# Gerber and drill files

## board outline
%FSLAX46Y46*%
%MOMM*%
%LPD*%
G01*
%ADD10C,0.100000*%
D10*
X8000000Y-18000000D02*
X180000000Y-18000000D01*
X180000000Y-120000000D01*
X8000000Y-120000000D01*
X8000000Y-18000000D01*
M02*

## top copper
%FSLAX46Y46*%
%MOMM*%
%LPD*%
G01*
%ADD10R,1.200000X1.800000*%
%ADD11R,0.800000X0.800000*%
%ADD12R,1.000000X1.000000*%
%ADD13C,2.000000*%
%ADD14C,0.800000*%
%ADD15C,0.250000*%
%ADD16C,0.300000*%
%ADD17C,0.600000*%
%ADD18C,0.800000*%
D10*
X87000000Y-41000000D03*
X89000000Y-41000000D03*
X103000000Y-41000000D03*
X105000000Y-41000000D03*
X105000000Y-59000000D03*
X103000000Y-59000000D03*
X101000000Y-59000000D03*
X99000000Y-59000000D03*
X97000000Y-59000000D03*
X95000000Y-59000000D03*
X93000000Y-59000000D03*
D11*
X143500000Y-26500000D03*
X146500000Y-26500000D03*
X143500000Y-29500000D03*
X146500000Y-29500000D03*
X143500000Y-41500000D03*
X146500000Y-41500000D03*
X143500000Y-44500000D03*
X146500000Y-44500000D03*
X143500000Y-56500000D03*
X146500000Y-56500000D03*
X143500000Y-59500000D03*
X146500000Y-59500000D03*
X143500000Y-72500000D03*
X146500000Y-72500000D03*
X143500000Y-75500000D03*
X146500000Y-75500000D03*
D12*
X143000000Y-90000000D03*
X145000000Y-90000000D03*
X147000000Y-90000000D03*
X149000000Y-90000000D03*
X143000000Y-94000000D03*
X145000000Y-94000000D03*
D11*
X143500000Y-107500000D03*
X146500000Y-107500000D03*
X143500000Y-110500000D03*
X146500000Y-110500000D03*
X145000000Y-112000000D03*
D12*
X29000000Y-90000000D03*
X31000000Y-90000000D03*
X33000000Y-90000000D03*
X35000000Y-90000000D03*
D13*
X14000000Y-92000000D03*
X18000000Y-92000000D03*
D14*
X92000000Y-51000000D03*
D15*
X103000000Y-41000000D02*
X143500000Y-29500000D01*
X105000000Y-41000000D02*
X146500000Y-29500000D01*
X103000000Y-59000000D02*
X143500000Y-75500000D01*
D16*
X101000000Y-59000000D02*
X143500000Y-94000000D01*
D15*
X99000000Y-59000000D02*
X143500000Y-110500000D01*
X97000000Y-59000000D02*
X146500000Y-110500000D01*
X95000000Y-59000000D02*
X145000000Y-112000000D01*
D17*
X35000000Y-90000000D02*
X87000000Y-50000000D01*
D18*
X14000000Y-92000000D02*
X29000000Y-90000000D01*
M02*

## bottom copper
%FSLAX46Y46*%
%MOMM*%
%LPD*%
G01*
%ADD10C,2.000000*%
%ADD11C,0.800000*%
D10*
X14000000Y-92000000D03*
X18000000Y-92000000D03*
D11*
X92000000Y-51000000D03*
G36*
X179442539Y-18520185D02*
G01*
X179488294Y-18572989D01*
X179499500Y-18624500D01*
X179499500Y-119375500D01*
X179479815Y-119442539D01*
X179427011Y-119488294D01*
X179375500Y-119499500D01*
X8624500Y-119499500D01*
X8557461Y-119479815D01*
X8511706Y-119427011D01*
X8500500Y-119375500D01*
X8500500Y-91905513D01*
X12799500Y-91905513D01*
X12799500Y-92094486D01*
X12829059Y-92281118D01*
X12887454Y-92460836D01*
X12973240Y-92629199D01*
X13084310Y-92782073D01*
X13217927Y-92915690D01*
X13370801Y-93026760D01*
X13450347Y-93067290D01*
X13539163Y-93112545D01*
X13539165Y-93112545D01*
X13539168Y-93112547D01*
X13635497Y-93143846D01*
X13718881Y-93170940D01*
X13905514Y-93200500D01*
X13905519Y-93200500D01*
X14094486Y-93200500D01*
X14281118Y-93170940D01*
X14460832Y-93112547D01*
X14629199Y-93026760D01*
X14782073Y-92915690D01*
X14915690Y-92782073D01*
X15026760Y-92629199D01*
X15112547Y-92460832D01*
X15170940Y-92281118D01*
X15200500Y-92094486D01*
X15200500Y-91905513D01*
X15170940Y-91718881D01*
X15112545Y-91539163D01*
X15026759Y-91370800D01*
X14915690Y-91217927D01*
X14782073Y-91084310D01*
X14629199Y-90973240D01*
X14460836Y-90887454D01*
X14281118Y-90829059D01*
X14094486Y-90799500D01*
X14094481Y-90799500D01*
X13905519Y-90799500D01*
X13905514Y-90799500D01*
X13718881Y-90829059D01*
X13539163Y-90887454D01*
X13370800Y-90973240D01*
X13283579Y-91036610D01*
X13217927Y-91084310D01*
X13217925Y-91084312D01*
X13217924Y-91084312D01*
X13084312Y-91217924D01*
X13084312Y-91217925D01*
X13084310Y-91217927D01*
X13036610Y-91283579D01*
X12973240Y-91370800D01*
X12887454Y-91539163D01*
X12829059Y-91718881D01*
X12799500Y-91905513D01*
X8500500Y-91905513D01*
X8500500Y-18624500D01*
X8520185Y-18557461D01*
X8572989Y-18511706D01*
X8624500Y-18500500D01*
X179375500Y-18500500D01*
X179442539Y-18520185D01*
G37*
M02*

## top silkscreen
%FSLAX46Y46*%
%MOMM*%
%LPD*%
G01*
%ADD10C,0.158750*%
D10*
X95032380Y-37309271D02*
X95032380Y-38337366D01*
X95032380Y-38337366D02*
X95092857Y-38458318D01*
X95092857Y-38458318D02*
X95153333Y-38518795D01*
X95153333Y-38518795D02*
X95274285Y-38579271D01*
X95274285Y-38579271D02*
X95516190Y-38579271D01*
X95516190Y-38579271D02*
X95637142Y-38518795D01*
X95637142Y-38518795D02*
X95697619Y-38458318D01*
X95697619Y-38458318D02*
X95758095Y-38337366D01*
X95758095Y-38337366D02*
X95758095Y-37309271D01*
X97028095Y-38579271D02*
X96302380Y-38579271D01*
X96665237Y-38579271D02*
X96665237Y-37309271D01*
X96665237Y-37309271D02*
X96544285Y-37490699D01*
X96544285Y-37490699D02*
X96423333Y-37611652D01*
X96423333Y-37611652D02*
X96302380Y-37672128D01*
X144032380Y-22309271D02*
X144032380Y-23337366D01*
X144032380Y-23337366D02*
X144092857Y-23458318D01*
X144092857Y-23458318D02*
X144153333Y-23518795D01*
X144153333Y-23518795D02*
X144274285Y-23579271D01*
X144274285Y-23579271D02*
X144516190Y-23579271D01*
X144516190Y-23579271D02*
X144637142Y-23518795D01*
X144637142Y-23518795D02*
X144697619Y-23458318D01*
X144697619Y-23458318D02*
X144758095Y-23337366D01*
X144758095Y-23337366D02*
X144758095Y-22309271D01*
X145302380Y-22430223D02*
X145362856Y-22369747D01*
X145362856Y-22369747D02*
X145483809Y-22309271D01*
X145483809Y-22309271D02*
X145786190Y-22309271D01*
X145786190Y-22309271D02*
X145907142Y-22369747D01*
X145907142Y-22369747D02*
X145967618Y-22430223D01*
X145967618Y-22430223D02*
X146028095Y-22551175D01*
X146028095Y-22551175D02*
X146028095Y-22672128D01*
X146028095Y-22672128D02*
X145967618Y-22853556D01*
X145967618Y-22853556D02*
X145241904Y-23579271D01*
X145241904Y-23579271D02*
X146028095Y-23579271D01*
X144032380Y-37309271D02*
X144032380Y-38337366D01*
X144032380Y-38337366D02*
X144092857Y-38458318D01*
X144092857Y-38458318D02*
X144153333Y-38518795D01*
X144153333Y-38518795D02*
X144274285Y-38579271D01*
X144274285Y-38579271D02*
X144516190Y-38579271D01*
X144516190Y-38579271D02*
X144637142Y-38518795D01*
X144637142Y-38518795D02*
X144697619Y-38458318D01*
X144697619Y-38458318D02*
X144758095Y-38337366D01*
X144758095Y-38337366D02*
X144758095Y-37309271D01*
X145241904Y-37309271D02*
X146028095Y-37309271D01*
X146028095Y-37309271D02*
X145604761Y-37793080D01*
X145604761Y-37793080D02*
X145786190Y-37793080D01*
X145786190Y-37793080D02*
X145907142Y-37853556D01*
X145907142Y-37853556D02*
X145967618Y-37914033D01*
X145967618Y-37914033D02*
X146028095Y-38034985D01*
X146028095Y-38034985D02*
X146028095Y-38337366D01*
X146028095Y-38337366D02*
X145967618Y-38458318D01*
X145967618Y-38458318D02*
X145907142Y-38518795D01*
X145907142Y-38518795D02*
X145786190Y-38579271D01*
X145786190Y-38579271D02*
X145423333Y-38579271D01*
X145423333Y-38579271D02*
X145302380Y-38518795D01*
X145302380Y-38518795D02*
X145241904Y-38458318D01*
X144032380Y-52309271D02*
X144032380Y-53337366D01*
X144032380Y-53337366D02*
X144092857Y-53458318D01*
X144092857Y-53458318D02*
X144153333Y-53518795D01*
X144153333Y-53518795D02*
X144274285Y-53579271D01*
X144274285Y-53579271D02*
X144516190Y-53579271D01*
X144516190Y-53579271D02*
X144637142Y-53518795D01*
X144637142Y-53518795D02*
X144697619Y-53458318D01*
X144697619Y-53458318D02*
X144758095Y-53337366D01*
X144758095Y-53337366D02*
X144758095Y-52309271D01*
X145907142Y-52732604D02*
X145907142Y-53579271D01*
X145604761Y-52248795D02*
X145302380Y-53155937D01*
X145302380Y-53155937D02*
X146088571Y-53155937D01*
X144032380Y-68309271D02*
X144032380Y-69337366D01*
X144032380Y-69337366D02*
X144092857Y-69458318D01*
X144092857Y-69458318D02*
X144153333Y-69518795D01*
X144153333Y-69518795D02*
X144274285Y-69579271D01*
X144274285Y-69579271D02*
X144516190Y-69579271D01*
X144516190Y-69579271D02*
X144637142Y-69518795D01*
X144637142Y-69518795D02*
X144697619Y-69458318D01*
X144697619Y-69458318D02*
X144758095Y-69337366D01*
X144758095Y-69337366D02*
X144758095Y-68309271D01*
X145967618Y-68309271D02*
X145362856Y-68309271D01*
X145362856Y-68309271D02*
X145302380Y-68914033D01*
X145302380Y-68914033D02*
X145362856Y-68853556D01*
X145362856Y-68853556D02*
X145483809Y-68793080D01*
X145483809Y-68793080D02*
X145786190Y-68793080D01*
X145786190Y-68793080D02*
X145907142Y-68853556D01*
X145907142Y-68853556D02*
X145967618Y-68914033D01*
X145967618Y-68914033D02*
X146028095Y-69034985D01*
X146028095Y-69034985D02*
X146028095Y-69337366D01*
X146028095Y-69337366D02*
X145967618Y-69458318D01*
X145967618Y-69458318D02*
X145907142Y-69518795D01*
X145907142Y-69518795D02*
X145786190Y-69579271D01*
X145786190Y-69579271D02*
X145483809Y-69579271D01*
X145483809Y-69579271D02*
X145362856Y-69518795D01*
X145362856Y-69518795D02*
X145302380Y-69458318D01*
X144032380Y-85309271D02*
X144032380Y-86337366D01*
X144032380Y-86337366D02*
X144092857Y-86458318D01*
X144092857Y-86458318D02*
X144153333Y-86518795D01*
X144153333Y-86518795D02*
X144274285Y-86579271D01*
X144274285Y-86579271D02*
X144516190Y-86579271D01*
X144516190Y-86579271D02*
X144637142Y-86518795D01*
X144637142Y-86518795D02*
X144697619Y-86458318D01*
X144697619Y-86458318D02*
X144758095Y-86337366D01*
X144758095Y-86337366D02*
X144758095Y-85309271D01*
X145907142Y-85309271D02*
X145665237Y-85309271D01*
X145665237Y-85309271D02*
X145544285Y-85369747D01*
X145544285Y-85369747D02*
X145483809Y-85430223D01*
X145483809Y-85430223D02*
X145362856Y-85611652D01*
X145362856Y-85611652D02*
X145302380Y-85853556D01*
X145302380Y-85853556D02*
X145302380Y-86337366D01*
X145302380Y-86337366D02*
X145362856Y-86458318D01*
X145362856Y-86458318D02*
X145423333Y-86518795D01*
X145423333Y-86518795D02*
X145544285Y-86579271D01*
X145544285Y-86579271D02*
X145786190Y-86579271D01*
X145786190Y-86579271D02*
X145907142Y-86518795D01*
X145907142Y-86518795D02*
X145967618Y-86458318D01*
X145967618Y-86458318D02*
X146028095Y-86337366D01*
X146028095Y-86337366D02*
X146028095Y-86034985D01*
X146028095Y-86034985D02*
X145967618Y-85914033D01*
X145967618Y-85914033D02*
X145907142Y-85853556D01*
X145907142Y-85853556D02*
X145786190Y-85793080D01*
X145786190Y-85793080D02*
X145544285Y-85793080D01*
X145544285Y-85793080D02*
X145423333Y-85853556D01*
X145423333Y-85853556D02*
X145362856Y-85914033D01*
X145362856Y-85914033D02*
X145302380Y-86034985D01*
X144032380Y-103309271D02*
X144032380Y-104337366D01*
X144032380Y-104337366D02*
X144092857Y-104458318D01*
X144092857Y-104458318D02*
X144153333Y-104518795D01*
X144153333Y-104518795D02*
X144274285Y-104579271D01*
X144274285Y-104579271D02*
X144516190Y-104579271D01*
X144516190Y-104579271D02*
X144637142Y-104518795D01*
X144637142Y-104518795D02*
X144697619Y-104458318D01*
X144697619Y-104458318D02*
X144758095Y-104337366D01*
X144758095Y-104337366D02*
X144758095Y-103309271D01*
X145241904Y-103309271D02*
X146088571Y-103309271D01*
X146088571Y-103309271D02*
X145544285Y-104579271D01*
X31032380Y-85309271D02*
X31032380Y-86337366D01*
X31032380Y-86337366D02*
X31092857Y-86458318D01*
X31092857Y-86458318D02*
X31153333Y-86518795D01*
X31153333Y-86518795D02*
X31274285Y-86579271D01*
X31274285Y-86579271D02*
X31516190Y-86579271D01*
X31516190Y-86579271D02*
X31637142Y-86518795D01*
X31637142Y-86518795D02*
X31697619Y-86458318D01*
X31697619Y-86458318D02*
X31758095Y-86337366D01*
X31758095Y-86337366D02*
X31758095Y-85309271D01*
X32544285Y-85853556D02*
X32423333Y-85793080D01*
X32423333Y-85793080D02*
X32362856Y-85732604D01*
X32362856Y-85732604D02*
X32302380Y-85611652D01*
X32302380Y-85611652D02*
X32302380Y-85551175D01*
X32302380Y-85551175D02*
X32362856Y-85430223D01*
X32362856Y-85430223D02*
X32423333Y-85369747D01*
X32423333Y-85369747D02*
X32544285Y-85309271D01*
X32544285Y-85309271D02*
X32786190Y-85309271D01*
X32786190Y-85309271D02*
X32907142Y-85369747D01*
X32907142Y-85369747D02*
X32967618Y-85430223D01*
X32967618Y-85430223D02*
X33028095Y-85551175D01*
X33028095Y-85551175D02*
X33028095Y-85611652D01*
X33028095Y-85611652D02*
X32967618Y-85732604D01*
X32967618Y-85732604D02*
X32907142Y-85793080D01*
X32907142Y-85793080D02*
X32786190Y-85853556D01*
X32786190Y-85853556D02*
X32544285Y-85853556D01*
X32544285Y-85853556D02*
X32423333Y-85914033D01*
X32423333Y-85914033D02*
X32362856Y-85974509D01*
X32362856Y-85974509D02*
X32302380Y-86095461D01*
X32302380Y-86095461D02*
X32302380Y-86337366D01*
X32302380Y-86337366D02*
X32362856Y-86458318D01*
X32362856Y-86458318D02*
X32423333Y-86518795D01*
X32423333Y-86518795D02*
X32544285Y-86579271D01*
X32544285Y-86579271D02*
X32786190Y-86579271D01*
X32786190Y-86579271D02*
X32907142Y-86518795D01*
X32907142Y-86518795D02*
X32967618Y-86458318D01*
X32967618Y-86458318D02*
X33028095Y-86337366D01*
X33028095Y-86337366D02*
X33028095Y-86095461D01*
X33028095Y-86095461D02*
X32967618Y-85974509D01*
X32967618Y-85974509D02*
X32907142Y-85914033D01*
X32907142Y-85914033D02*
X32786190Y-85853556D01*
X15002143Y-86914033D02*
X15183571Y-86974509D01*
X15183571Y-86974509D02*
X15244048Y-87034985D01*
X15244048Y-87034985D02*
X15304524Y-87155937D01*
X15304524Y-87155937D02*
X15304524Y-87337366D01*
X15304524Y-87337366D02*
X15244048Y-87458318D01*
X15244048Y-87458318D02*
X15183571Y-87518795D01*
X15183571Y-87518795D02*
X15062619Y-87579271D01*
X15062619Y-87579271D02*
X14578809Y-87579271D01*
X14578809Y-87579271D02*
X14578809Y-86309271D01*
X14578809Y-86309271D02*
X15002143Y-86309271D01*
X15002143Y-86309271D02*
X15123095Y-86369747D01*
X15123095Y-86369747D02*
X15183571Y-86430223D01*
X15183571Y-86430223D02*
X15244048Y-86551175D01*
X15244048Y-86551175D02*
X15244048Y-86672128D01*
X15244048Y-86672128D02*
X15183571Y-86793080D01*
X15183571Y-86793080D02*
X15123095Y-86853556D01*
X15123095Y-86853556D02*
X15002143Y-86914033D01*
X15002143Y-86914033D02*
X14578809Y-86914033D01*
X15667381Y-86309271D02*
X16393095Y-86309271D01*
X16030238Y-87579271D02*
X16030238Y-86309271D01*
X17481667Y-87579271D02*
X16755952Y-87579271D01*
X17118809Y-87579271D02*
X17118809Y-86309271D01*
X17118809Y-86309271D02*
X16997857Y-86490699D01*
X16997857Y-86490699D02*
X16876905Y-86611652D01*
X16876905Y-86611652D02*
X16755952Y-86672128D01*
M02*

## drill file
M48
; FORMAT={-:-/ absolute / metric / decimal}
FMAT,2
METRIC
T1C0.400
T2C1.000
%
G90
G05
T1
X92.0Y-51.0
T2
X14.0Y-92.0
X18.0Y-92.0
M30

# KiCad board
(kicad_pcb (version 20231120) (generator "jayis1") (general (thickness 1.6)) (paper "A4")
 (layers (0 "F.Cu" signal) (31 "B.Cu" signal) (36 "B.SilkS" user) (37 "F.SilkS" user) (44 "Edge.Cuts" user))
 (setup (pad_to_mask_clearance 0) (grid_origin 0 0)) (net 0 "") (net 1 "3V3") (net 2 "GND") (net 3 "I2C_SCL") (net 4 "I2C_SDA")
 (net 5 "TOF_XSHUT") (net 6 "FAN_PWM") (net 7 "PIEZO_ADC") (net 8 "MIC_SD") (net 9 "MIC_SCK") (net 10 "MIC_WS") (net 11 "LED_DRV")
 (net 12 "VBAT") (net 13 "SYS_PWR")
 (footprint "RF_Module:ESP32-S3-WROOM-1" (layer "F.Cu") (at 96 50) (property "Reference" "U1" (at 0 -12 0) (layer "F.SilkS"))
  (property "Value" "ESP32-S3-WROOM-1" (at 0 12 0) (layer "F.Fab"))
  (pad "1" smd rect (at -9 -9) (size 1.2 1.8) (layers "F.Cu" "F.Mask") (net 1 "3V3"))
  (pad "2" smd rect (at -7 -9) (size 1.2 1.8) (layers "F.Cu" "F.Mask") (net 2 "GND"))
  (pad "3" smd rect (at 7 -9) (size 1.2 1.8) (layers "F.Cu" "F.Mask") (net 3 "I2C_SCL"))
  (pad "4" smd rect (at 9 -9) (size 1.2 1.8) (layers "F.Cu" "F.Mask") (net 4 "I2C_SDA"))
  (pad "5" smd rect (at 9 9) (size 1.2 1.8) (layers "F.Cu" "F.Mask") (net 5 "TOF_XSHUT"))
  (pad "6" smd rect (at 7 9) (size 1.2 1.8) (layers "F.Cu" "F.Mask") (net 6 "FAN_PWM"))
  (pad "7" smd rect (at 5 9) (size 1.2 1.8) (layers "F.Cu" "F.Mask") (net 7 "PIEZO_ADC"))
  (pad "8" smd rect (at 3 9) (size 1.2 1.8) (layers "F.Cu" "F.Mask") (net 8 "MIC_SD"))
  (pad "9" smd rect (at 1 9) (size 1.2 1.8) (layers "F.Cu" "F.Mask") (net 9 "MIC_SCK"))
  (pad "10" smd rect (at -1 9) (size 1.2 1.8) (layers "F.Cu" "F.Mask") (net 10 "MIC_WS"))
  (pad "11" smd rect (at -3 9) (size 1.2 1.8) (layers "F.Cu" "F.Mask") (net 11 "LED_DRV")))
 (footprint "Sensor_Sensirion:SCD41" (layer "F.Cu") (at 145 28) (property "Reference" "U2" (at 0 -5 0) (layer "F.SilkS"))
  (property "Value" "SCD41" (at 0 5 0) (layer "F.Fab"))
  (pad "1" smd rect (at -1.5 -1.5) (size 0.8 0.8) (layers "F.Cu" "F.Mask") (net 1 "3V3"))
  (pad "2" smd rect (at 1.5 -1.5) (size 0.8 0.8) (layers "F.Cu" "F.Mask") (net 2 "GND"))
  (pad "3" smd rect (at -1.5 1.5) (size 0.8 0.8) (layers "F.Cu" "F.Mask") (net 3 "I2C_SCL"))
  (pad "4" smd rect (at 1.5 1.5) (size 0.8 0.8) (layers "F.Cu" "F.Mask") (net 4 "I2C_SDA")))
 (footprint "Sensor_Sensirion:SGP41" (layer "F.Cu") (at 145 43) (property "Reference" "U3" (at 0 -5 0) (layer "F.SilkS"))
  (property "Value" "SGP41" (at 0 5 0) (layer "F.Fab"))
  (pad "1" smd rect (at -1.5 -1.5) (size 0.8 0.8) (layers "F.Cu" "F.Mask") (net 1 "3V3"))
  (pad "2" smd rect (at 1.5 -1.5) (size 0.8 0.8) (layers "F.Cu" "F.Mask") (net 2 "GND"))
  (pad "3" smd rect (at -1.5 1.5) (size 0.8 0.8) (layers "F.Cu" "F.Mask") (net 3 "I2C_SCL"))
  (pad "4" smd rect (at 1.5 1.5) (size 0.8 0.8) (layers "F.Cu" "F.Mask") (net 4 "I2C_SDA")))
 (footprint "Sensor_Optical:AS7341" (layer "F.Cu") (at 145 58) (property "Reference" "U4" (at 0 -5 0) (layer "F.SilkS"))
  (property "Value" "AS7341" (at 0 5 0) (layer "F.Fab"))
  (pad "1" smd rect (at -1.5 -1.5) (size 0.8 0.8) (layers "F.Cu" "F.Mask") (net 1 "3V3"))
  (pad "2" smd rect (at 1.5 -1.5) (size 0.8 0.8) (layers "F.Cu" "F.Mask") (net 2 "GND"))
  (pad "3" smd rect (at -1.5 1.5) (size 0.8 0.8) (layers "F.Cu" "F.Mask") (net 3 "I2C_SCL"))
  (pad "4" smd rect (at 1.5 1.5) (size 0.8 0.8) (layers "F.Cu" "F.Mask") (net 4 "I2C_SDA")))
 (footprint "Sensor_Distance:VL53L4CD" (layer "F.Cu") (at 145 74) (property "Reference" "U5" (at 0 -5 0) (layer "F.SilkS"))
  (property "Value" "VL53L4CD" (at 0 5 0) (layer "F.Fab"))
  (pad "1" smd rect (at -1.5 -1.5) (size 0.8 0.8) (layers "F.Cu" "F.Mask") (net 1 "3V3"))
  (pad "2" smd rect (at 1.5 -1.5) (size 0.8 0.8) (layers "F.Cu" "F.Mask") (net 2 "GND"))
  (pad "3" smd rect (at -1.5 1.5) (size 0.8 0.8) (layers "F.Cu" "F.Mask") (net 3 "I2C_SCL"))
  (pad "4" smd rect (at 1.5 1.5) (size 0.8 0.8) (layers "F.Cu" "F.Mask") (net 4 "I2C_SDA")))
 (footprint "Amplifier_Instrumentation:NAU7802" (layer "F.Cu") (at 145 92) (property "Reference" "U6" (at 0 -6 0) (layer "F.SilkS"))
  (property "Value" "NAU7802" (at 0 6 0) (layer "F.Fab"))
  (pad "1" smd rect (at -2 -2) (size 1 1) (layers "F.Cu" "F.Mask") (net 1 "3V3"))
  (pad "2" smd rect (at 0 -2) (size 1 1) (layers "F.Cu" "F.Mask") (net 2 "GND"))
  (pad "3" smd rect (at 2 -2) (size 1 1) (layers "F.Cu" "F.Mask") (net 3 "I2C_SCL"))
  (pad "4" smd rect (at 4 -2) (size 1 1) (layers "F.Cu" "F.Mask") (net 4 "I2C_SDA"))
  (pad "5" smd rect (at -2 2) (size 1 1) (layers "F.Cu" "F.Mask") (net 7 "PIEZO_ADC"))
  (pad "6" smd rect (at 0 2) (size 1 1) (layers "F.Cu" "F.Mask") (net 2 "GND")))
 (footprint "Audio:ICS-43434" (layer "F.Cu") (at 145 109) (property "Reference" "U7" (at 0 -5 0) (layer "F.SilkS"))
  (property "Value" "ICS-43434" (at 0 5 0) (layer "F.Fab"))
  (pad "1" smd rect (at -1.5 -1.5) (size 0.8 0.8) (layers "F.Cu" "F.Mask") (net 1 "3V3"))
  (pad "2" smd rect (at 1.5 -1.5) (size 0.8 0.8) (layers "F.Cu" "F.Mask") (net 2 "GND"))
  (pad "3" smd rect (at -1.5 1.5) (size 0.8 0.8) (layers "F.Cu" "F.Mask") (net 8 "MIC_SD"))
  (pad "4" smd rect (at 1.5 1.5) (size 0.8 0.8) (layers "F.Cu" "F.Mask") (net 9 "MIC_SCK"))
  (pad "5" smd rect (at 0 3.0) (size 0.8 0.8) (layers "F.Cu" "F.Mask") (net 10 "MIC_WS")))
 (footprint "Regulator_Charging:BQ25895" (layer "F.Cu") (at 32 92) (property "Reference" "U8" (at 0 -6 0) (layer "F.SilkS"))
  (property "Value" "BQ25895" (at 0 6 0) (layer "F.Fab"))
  (pad "1" smd rect (at -3 -2) (size 1 1) (layers "F.Cu" "F.Mask") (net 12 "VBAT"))
  (pad "2" smd rect (at -1 -2) (size 1 1) (layers "F.Cu" "F.Mask") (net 12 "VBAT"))
  (pad "3" smd rect (at 1 -2) (size 1 1) (layers "F.Cu" "F.Mask") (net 2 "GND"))
  (pad "4" smd rect (at 3 -2) (size 1 1) (layers "F.Cu" "F.Mask") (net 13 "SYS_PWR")))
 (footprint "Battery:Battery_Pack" (layer "F.Cu") (at 16 92) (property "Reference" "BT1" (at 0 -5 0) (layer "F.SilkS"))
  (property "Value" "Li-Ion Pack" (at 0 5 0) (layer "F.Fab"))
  (pad "1" thru_hole circle (at -2 0) (size 2 2) (drill 1.0) (layers *.Cu *.Mask) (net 12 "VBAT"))
  (pad "2" thru_hole circle (at 2 0) (size 2 2) (drill 1.0) (layers *.Cu *.Mask) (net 2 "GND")))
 (gr_rect (start 8 18) (end 180 120) (stroke (width 0.1) (type default)) (fill none) (layer "Edge.Cuts"))
 (segment (start 103 41) (end 143.5 29.5) (width 0.25) (layer "F.Cu") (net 3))
 (segment (start 105 41) (end 146.5 29.5) (width 0.25) (layer "F.Cu") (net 4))
 (segment (start 103 59) (end 143.5 75.5) (width 0.25) (layer "F.Cu") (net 5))
 (segment (start 101 59) (end 143.5 94.0) (width 0.30) (layer "F.Cu") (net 7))
 (segment (start 99 59) (end 143.5 110.5) (width 0.25) (layer "F.Cu") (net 8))
 (segment (start 97 59) (end 146.5 110.5) (width 0.25) (layer "F.Cu") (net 9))
 (segment (start 95 59) (end 145 112.0) (width 0.25) (layer "F.Cu") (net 10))
 (segment (start 35 90) (end 87 50) (width 0.6) (layer "F.Cu") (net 13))
 (segment (start 14 92) (end 29 90) (width 0.8) (layer "F.Cu") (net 12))
 (via (at 92 51) (size 0.8) (drill 0.4) (layers "F.Cu" "B.Cu") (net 2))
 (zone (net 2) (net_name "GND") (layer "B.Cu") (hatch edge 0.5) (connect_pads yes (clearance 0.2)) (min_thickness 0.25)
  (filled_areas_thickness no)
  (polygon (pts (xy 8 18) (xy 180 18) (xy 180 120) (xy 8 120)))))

